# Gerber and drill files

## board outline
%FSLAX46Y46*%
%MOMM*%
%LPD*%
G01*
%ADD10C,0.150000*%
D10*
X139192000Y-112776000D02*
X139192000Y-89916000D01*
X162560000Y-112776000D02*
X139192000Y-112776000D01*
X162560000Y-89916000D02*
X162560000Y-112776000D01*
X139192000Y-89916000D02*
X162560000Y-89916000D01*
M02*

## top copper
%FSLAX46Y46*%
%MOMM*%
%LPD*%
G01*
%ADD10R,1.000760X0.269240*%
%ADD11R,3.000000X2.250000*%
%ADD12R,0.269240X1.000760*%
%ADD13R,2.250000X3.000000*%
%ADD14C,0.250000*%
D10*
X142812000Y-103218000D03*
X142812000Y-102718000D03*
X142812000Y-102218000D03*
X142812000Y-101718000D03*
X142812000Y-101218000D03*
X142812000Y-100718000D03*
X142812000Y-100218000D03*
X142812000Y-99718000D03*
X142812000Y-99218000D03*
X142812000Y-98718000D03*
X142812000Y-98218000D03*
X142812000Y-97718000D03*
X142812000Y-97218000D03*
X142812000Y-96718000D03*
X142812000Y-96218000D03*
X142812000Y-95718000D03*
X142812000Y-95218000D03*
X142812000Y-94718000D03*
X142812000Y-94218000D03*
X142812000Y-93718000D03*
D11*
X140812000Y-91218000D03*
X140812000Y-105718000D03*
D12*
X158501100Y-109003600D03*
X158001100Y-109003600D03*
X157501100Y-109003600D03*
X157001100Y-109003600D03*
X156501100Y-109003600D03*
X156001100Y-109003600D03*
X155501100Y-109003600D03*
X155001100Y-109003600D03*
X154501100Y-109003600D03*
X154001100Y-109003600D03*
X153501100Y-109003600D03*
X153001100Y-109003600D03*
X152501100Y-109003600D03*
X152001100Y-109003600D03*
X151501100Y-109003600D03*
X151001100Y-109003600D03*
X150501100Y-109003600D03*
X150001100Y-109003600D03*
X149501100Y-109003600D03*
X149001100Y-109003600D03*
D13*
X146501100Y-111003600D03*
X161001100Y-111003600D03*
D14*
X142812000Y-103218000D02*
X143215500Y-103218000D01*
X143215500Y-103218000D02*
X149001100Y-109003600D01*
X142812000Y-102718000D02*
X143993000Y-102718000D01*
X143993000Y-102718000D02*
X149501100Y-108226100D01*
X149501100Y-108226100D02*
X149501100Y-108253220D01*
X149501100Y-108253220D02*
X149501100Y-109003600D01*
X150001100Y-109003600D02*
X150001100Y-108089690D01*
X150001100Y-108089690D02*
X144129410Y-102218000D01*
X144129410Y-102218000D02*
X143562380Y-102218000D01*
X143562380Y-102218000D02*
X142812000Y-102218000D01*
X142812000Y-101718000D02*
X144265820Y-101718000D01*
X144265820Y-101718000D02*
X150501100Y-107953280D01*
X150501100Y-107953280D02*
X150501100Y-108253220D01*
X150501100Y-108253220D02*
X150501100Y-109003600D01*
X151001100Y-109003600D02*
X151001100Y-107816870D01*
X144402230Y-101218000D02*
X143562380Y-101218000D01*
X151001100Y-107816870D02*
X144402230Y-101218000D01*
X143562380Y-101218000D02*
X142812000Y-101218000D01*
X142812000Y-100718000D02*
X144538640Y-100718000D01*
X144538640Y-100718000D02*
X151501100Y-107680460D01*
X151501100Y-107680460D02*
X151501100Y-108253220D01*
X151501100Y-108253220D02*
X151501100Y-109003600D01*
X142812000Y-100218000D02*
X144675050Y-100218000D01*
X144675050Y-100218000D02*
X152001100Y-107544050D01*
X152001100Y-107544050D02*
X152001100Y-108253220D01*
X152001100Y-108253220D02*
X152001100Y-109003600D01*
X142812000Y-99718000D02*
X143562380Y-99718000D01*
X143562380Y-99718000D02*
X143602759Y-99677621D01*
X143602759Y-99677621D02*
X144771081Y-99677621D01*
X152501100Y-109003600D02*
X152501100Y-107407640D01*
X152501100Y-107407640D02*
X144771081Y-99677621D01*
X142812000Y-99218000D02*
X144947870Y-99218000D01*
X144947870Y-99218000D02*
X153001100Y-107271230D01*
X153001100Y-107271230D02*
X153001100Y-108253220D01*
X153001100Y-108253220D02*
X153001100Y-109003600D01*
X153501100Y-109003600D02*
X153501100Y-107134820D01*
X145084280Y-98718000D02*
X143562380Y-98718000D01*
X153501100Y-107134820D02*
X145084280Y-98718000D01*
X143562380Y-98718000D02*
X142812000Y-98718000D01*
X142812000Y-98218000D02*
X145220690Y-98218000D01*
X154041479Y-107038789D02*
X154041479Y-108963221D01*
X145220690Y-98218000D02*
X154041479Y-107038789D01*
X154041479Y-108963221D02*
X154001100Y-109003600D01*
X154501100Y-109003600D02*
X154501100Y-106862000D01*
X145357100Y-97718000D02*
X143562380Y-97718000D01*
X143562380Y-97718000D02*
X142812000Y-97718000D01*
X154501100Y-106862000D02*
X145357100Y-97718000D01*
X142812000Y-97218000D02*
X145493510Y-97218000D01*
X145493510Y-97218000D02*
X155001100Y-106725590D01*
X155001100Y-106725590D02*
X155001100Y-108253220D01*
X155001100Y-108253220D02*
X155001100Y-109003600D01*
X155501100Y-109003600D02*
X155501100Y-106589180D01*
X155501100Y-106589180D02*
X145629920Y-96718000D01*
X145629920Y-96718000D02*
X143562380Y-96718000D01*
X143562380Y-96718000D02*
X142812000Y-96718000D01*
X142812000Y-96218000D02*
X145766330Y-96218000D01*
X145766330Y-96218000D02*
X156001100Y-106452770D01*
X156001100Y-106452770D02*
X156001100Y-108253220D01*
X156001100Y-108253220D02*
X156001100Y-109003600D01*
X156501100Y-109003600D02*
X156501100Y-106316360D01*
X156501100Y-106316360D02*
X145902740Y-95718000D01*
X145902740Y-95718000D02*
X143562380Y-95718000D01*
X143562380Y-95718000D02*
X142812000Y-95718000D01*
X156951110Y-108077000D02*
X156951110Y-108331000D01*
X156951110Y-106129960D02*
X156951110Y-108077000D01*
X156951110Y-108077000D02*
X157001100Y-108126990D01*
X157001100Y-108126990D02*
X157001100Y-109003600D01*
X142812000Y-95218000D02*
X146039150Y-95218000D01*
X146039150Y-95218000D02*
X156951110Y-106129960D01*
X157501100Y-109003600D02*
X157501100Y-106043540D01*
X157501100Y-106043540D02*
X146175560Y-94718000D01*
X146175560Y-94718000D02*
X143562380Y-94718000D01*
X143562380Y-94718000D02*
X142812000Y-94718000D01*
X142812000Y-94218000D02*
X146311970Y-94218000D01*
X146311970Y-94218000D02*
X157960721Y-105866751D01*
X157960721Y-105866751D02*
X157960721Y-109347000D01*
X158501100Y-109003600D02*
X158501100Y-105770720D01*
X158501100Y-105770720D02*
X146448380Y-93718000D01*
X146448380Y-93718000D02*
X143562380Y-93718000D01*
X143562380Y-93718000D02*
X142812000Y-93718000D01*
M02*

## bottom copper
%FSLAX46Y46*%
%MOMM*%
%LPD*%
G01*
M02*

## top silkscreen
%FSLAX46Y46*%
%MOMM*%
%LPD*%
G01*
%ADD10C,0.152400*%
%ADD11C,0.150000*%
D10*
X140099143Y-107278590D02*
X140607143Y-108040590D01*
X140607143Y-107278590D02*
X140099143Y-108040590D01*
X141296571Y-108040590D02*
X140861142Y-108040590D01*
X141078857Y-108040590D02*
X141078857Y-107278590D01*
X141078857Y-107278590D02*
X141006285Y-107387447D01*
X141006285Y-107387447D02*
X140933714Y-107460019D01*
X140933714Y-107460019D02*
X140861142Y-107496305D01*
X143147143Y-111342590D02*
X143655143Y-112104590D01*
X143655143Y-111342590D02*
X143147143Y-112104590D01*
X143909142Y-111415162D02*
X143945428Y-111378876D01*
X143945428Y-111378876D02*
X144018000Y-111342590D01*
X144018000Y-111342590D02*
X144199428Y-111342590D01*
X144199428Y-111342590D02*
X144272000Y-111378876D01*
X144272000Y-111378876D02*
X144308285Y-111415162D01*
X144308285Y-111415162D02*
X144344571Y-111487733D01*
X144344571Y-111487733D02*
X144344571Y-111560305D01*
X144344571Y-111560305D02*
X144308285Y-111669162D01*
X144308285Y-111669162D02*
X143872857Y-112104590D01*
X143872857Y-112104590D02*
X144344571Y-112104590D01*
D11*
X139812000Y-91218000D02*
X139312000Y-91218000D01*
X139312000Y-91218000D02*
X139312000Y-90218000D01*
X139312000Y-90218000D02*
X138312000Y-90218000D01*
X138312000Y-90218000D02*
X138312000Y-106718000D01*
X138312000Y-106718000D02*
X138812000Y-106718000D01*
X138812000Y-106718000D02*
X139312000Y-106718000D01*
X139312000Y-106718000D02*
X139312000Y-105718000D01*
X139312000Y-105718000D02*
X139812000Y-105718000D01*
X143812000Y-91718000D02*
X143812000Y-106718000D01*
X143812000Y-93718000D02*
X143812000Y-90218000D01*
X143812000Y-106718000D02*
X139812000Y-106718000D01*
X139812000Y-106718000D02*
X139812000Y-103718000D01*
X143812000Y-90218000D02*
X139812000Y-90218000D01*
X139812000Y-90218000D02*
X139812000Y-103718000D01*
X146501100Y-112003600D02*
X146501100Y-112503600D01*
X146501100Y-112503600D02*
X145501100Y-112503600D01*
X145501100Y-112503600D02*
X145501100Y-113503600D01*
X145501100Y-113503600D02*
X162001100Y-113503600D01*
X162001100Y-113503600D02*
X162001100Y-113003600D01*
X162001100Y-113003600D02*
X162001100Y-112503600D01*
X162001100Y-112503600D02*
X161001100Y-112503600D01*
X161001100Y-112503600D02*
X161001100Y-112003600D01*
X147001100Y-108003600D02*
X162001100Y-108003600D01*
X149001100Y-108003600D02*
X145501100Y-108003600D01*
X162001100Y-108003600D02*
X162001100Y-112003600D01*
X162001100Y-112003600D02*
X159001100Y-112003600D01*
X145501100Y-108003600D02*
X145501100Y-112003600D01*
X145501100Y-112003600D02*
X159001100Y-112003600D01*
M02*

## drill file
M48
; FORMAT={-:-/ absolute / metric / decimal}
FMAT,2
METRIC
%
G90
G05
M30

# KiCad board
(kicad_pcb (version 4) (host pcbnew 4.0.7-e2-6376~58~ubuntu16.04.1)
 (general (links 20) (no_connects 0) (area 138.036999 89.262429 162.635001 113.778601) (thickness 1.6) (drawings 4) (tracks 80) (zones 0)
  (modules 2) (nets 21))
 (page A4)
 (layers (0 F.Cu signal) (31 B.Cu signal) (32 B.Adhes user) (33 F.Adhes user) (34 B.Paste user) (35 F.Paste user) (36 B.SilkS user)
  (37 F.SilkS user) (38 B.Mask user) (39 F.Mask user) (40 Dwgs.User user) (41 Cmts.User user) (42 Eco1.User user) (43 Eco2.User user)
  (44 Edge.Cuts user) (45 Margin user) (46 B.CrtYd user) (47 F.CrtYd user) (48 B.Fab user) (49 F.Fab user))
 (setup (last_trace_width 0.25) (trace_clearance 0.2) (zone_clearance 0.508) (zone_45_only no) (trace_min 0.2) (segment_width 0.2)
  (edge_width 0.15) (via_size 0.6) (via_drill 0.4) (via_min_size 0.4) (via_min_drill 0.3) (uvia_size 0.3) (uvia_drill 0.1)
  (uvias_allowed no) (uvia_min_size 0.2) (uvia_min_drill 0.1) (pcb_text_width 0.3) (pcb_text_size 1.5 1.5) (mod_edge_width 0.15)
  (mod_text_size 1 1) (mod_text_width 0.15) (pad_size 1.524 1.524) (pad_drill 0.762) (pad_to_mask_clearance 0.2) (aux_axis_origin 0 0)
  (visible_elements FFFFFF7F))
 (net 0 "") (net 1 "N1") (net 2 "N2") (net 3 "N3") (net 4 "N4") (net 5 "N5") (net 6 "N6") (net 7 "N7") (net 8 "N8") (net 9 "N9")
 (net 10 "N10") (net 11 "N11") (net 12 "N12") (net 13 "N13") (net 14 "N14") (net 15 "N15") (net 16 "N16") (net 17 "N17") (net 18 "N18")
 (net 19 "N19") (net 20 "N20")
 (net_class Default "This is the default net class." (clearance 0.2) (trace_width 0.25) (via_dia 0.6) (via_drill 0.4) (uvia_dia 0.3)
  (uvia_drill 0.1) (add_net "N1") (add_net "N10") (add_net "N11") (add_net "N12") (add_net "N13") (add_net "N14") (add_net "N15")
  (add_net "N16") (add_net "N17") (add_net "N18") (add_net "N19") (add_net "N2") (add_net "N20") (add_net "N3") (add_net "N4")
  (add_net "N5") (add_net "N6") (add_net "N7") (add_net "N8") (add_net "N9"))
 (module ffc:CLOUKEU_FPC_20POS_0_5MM (layer F.Cu) (at 146.812 93.218 270)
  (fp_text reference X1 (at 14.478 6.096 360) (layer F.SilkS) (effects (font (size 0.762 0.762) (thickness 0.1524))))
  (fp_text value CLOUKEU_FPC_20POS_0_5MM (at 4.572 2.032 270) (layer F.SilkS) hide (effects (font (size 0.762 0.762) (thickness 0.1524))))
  (fp_line (start -2 7) (end -2 7.5) (layer F.SilkS) (width 0.15))
  (fp_line (start -2 7.5) (end -3 7.5) (layer F.SilkS) (width 0.15))
  (fp_line (start -3 7.5) (end -3 8.5) (layer F.SilkS) (width 0.15))
  (fp_line (start -3 8.5) (end 13.5 8.5) (layer F.SilkS) (width 0.15))
  (fp_line (start 13.5 8.5) (end 13.5 8) (layer F.SilkS) (width 0.15))
  (fp_line (start 13.5 8) (end 13.5 7.5) (layer F.SilkS) (width 0.15))
  (fp_line (start 13.5 7.5) (end 12.5 7.5) (layer F.SilkS) (width 0.15))
  (fp_line (start 12.5 7.5) (end 12.5 7) (layer F.SilkS) (width 0.15))
  (fp_line (start -1.5 3) (end 13.5 3) (layer F.SilkS) (width 0.15))
  (fp_line (start 0.5 3) (end -3 3) (layer F.SilkS) (width 0.15))
  (fp_line (start 13.5 3) (end 13.5 7) (layer F.SilkS) (width 0.15))
  (fp_line (start 13.5 7) (end 10.5 7) (layer F.SilkS) (width 0.15))
  (fp_line (start -3 3) (end -3 7) (layer F.SilkS) (width 0.15))
  (fp_line (start -3 7) (end 10.5 7) (layer F.SilkS) (width 0.15))
  (pad 1 smd rect (at 10 4 90) (size 0.26924 1.00076) (layers F.Cu F.Paste F.Mask) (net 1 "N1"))
  (pad 2 smd rect (at 9.5 4 90) (size 0.26924 1.00076) (layers F.Cu F.Paste F.Mask) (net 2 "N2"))
  (pad 3 smd rect (at 9 4 90) (size 0.26924 1.00076) (layers F.Cu F.Paste F.Mask) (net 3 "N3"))
  (pad 4 smd rect (at 8.5 4 90) (size 0.26924 1.00076) (layers F.Cu F.Paste F.Mask) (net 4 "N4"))
  (pad 5 smd rect (at 8 4 90) (size 0.26924 1.00076) (layers F.Cu F.Paste F.Mask) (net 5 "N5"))
  (pad 6 smd rect (at 7.5 4 90) (size 0.26924 1.00076) (layers F.Cu F.Paste F.Mask) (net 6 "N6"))
  (pad 7 smd rect (at 7 4 90) (size 0.26924 1.00076) (layers F.Cu F.Paste F.Mask) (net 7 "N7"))
  (pad 8 smd rect (at 6.5 4 90) (size 0.26924 1.00076) (layers F.Cu F.Paste F.Mask) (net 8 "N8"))
  (pad 9 smd rect (at 6 4 90) (size 0.26924 1.00076) (layers F.Cu F.Paste F.Mask) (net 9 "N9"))
  (pad 10 smd rect (at 5.5 4 90) (size 0.26924 1.00076) (layers F.Cu F.Paste F.Mask) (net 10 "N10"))
  (pad 11 smd rect (at 5 4 90) (size 0.26924 1.00076) (layers F.Cu F.Paste F.Mask) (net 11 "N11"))
  (pad 12 smd rect (at 4.5 4 90) (size 0.26924 1.00076) (layers F.Cu F.Paste F.Mask) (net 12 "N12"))
  (pad 13 smd rect (at 4 4 90) (size 0.26924 1.00076) (layers F.Cu F.Paste F.Mask) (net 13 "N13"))
  (pad 14 smd rect (at 3.5 4 90) (size 0.26924 1.00076) (layers F.Cu F.Paste F.Mask) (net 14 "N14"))
  (pad 15 smd rect (at 3 4 90) (size 0.26924 1.00076) (layers F.Cu F.Paste F.Mask) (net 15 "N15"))
  (pad 16 smd rect (at 2.5 4 90) (size 0.26924 1.00076) (layers F.Cu F.Paste F.Mask) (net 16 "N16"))
  (pad 17 smd rect (at 2 4 90) (size 0.26924 1.00076) (layers F.Cu F.Paste F.Mask) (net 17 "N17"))
  (pad 18 smd rect (at 1.5 4 90) (size 0.26924 1.00076) (layers F.Cu F.Paste F.Mask) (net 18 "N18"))
  (pad 19 smd rect (at 1 4 90) (size 0.26924 1.00076) (layers F.Cu F.Paste F.Mask) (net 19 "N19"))
  (pad 20 smd rect (at 0.5 4 90) (size 0.26924 1.00076) (layers F.Cu F.Paste F.Mask) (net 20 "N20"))
  (pad M1 smd rect (at -2 6 270) (size 2.25 3) (layers F.Cu F.Paste F.Mask))
  (pad M2 smd rect (at 12.5 6 270) (size 2.25 3) (layers F.Cu F.Paste F.Mask)))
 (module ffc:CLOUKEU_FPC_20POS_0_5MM (layer F.Cu) (at 148.5011 105.0036)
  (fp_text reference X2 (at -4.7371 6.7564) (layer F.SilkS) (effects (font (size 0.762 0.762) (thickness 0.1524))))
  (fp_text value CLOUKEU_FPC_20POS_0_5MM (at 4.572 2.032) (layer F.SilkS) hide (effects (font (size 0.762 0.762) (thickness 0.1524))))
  (fp_line (start -2 7) (end -2 7.5) (layer F.SilkS) (width 0.15))
  (fp_line (start -2 7.5) (end -3 7.5) (layer F.SilkS) (width 0.15))
  (fp_line (start -3 7.5) (end -3 8.5) (layer F.SilkS) (width 0.15))
  (fp_line (start -3 8.5) (end 13.5 8.5) (layer F.SilkS) (width 0.15))
  (fp_line (start 13.5 8.5) (end 13.5 8) (layer F.SilkS) (width 0.15))
  (fp_line (start 13.5 8) (end 13.5 7.5) (layer F.SilkS) (width 0.15))
  (fp_line (start 13.5 7.5) (end 12.5 7.5) (layer F.SilkS) (width 0.15))
  (fp_line (start 12.5 7.5) (end 12.5 7) (layer F.SilkS) (width 0.15))
  (fp_line (start -1.5 3) (end 13.5 3) (layer F.SilkS) (width 0.15))
  (fp_line (start 0.5 3) (end -3 3) (layer F.SilkS) (width 0.15))
  (fp_line (start 13.5 3) (end 13.5 7) (layer F.SilkS) (width 0.15))
  (fp_line (start 13.5 7) (end 10.5 7) (layer F.SilkS) (width 0.15))
  (fp_line (start -3 3) (end -3 7) (layer F.SilkS) (width 0.15))
  (fp_line (start -3 7) (end 10.5 7) (layer F.SilkS) (width 0.15))
  (pad 1 smd rect (at 10 4 180) (size 0.26924 1.00076) (layers F.Cu F.Paste F.Mask) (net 20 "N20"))
  (pad 2 smd rect (at 9.5 4 180) (size 0.26924 1.00076) (layers F.Cu F.Paste F.Mask) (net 19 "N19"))
  (pad 3 smd rect (at 9 4 180) (size 0.26924 1.00076) (layers F.Cu F.Paste F.Mask) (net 18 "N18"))
  (pad 4 smd rect (at 8.5 4 180) (size 0.26924 1.00076) (layers F.Cu F.Paste F.Mask) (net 17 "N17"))
  (pad 5 smd rect (at 8 4 180) (size 0.26924 1.00076) (layers F.Cu F.Paste F.Mask) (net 16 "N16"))
  (pad 6 smd rect (at 7.5 4 180) (size 0.26924 1.00076) (layers F.Cu F.Paste F.Mask) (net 15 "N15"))
  (pad 7 smd rect (at 7 4 180) (size 0.26924 1.00076) (layers F.Cu F.Paste F.Mask) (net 14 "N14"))
  (pad 8 smd rect (at 6.5 4 180) (size 0.26924 1.00076) (layers F.Cu F.Paste F.Mask) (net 13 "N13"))
  (pad 9 smd rect (at 6 4 180) (size 0.26924 1.00076) (layers F.Cu F.Paste F.Mask) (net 12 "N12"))
  (pad 10 smd rect (at 5.5 4 180) (size 0.26924 1.00076) (layers F.Cu F.Paste F.Mask) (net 11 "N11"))
  (pad 11 smd rect (at 5 4 180) (size 0.26924 1.00076) (layers F.Cu F.Paste F.Mask) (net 10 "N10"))
  (pad 12 smd rect (at 4.5 4 180) (size 0.26924 1.00076) (layers F.Cu F.Paste F.Mask) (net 9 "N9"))
  (pad 13 smd rect (at 4 4 180) (size 0.26924 1.00076) (layers F.Cu F.Paste F.Mask) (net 8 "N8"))
  (pad 14 smd rect (at 3.5 4 180) (size 0.26924 1.00076) (layers F.Cu F.Paste F.Mask) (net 7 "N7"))
  (pad 15 smd rect (at 3 4 180) (size 0.26924 1.00076) (layers F.Cu F.Paste F.Mask) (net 6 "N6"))
  (pad 16 smd rect (at 2.5 4 180) (size 0.26924 1.00076) (layers F.Cu F.Paste F.Mask) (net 5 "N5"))
  (pad 17 smd rect (at 2 4 180) (size 0.26924 1.00076) (layers F.Cu F.Paste F.Mask) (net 4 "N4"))
  (pad 18 smd rect (at 1.5 4 180) (size 0.26924 1.00076) (layers F.Cu F.Paste F.Mask) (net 3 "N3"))
  (pad 19 smd rect (at 1 4 180) (size 0.26924 1.00076) (layers F.Cu F.Paste F.Mask) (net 2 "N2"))
  (pad 20 smd rect (at 0.5 4 180) (size 0.26924 1.00076) (layers F.Cu F.Paste F.Mask) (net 1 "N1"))
  (pad M1 smd rect (at -2 6) (size 2.25 3) (layers F.Cu F.Paste F.Mask))
  (pad M2 smd rect (at 12.5 6) (size 2.25 3) (layers F.Cu F.Paste F.Mask)))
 (gr_line (start 139.192 112.776) (end 139.192 89.916) (angle 90) (layer Edge.Cuts) (width 0.15))
 (gr_line (start 162.56 112.776) (end 139.192 112.776) (angle 90) (layer Edge.Cuts) (width 0.15))
 (gr_line (start 162.56 89.916) (end 162.56 112.776) (angle 90) (layer Edge.Cuts) (width 0.15))
 (gr_line (start 139.192 89.916) (end 162.56 89.916) (angle 90) (layer Edge.Cuts) (width 0.15))
 (segment (start 142.812 103.218) (end 143.2155 103.218) (width 0.25) (layer F.Cu) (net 1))
 (segment (start 143.2155 103.218) (end 149.0011 109.0036) (width 0.25) (layer F.Cu) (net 1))
 (segment (start 142.812 102.718) (end 143.993 102.718) (width 0.25) (layer F.Cu) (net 2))
 (segment (start 143.993 102.718) (end 149.5011 108.2261) (width 0.25) (layer F.Cu) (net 2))
 (segment (start 149.5011 108.2261) (end 149.5011 108.25322) (width 0.25) (layer F.Cu) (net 2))
 (segment (start 149.5011 108.25322) (end 149.5011 109.0036) (width 0.25) (layer F.Cu) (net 2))
 (segment (start 150.0011 109.0036) (end 150.0011 108.08969) (width 0.25) (layer F.Cu) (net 3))
 (segment (start 150.0011 108.08969) (end 144.12941 102.218) (width 0.25) (layer F.Cu) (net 3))
 (segment (start 144.12941 102.218) (end 143.56238 102.218) (width 0.25) (layer F.Cu) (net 3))
 (segment (start 143.56238 102.218) (end 142.812 102.218) (width 0.25) (layer F.Cu) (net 3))
 (segment (start 142.812 101.718) (end 144.26582 101.718) (width 0.25) (layer F.Cu) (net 4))
 (segment (start 144.26582 101.718) (end 150.5011 107.95328) (width 0.25) (layer F.Cu) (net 4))
 (segment (start 150.5011 107.95328) (end 150.5011 108.25322) (width 0.25) (layer F.Cu) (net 4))
 (segment (start 150.5011 108.25322) (end 150.5011 109.0036) (width 0.25) (layer F.Cu) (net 4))
 (segment (start 151.0011 109.0036) (end 151.0011 107.81687) (width 0.25) (layer F.Cu) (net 5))
 (segment (start 144.40223 101.218) (end 143.56238 101.218) (width 0.25) (layer F.Cu) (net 5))
 (segment (start 151.0011 107.81687) (end 144.40223 101.218) (width 0.25) (layer F.Cu) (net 5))
 (segment (start 143.56238 101.218) (end 142.812 101.218) (width 0.25) (layer F.Cu) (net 5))
 (segment (start 142.812 100.718) (end 144.53864 100.718) (width 0.25) (layer F.Cu) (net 6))
 (segment (start 144.53864 100.718) (end 151.5011 107.68046) (width 0.25) (layer F.Cu) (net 6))
 (segment (start 151.5011 107.68046) (end 151.5011 108.25322) (width 0.25) (layer F.Cu) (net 6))
 (segment (start 151.5011 108.25322) (end 151.5011 109.0036) (width 0.25) (layer F.Cu) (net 6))
 (segment (start 142.812 100.218) (end 144.67505 100.218) (width 0.25) (layer F.Cu) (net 7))
 (segment (start 144.67505 100.218) (end 152.0011 107.54405) (width 0.25) (layer F.Cu) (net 7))
 (segment (start 152.0011 107.54405) (end 152.0011 108.25322) (width 0.25) (layer F.Cu) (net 7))
 (segment (start 152.0011 108.25322) (end 152.0011 109.0036) (width 0.25) (layer F.Cu) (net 7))
 (segment (start 142.812 99.718) (end 143.56238 99.718) (width 0.25) (layer F.Cu) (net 8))
 (segment (start 143.56238 99.718) (end 143.602759 99.677621) (width 0.25) (layer F.Cu) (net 8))
 (segment (start 143.602759 99.677621) (end 144.771081 99.677621) (width 0.25) (layer F.Cu) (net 8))
 (segment (start 152.5011 109.0036) (end 152.5011 107.40764) (width 0.25) (layer F.Cu) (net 8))
 (segment (start 152.5011 107.40764) (end 144.771081 99.677621) (width 0.25) (layer F.Cu) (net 8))
 (segment (start 142.812 99.218) (end 144.94787 99.218) (width 0.25) (layer F.Cu) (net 9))
 (segment (start 144.94787 99.218) (end 153.0011 107.27123) (width 0.25) (layer F.Cu) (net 9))
 (segment (start 153.0011 107.27123) (end 153.0011 108.25322) (width 0.25) (layer F.Cu) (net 9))
 (segment (start 153.0011 108.25322) (end 153.0011 109.0036) (width 0.25) (layer F.Cu) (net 9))
 (segment (start 153.5011 109.0036) (end 153.5011 107.13482) (width 0.25) (layer F.Cu) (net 10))
 (segment (start 145.08428 98.718) (end 143.56238 98.718) (width 0.25) (layer F.Cu) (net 10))
 (segment (start 153.5011 107.13482) (end 145.08428 98.718) (width 0.25) (layer F.Cu) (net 10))
 (segment (start 143.56238 98.718) (end 142.812 98.718) (width 0.25) (layer F.Cu) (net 10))
 (segment (start 142.812 98.218) (end 145.22069 98.218) (width 0.25) (layer F.Cu) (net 11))
 (segment (start 154.041479 107.038789) (end 154.041479 108.963221) (width 0.25) (layer F.Cu) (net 11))
 (segment (start 145.22069 98.218) (end 154.041479 107.038789) (width 0.25) (layer F.Cu) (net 11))
 (segment (start 154.041479 108.963221) (end 154.0011 109.0036) (width 0.25) (layer F.Cu) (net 11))
 (segment (start 154.5011 109.0036) (end 154.5011 106.862) (width 0.25) (layer F.Cu) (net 12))
 (segment (start 145.3571 97.718) (end 143.56238 97.718) (width 0.25) (layer F.Cu) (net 12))
 (segment (start 143.56238 97.718) (end 142.812 97.718) (width 0.25) (layer F.Cu) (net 12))
 (segment (start 154.5011 106.862) (end 145.3571 97.718) (width 0.25) (layer F.Cu) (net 12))
 (segment (start 142.812 97.218) (end 145.49351 97.218) (width 0.25) (layer F.Cu) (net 13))
 (segment (start 145.49351 97.218) (end 155.0011 106.72559) (width 0.25) (layer F.Cu) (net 13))
 (segment (start 155.0011 106.72559) (end 155.0011 108.25322) (width 0.25) (layer F.Cu) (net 13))
 (segment (start 155.0011 108.25322) (end 155.0011 109.0036) (width 0.25) (layer F.Cu) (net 13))
 (segment (start 155.5011 109.0036) (end 155.5011 106.58918) (width 0.25) (layer F.Cu) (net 14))
 (segment (start 155.5011 106.58918) (end 145.62992 96.718) (width 0.25) (layer F.Cu) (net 14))
 (segment (start 145.62992 96.718) (end 143.56238 96.718) (width 0.25) (layer F.Cu) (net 14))
 (segment (start 143.56238 96.718) (end 142.812 96.718) (width 0.25) (layer F.Cu) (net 14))
 (segment (start 142.812 96.218) (end 145.76633 96.218) (width 0.25) (layer F.Cu) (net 15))
 (segment (start 145.76633 96.218) (end 156.0011 106.45277) (width 0.25) (layer F.Cu) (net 15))
 (segment (start 156.0011 106.45277) (end 156.0011 108.25322) (width 0.25) (layer F.Cu) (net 15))
 (segment (start 156.0011 108.25322) (end 156.0011 109.0036) (width 0.25) (layer F.Cu) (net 15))
 (segment (start 156.5011 109.0036) (end 156.5011 106.31636) (width 0.25) (layer F.Cu) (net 16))
 (segment (start 156.5011 106.31636) (end 145.90274 95.718) (width 0.25) (layer F.Cu) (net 16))
 (segment (start 145.90274 95.718) (end 143.56238 95.718) (width 0.25) (layer F.Cu) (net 16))
 (segment (start 143.56238 95.718) (end 142.812 95.718) (width 0.25) (layer F.Cu) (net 16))
 (segment (start 156.95111 108.077) (end 156.95111 108.331) (width 0.25) (layer F.Cu) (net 17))
 (segment (start 156.95111 106.12996) (end 156.95111 108.077) (width 0.25) (layer F.Cu) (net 17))
 (segment (start 156.95111 108.077) (end 157.0011 108.12699) (width 0.25) (layer F.Cu) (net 17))
 (segment (start 157.0011 108.12699) (end 157.0011 109.0036) (width 0.25) (layer F.Cu) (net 17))
 (segment (start 142.812 95.218) (end 146.03915 95.218) (width 0.25) (layer F.Cu) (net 17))
 (segment (start 146.03915 95.218) (end 156.95111 106.12996) (width 0.25) (layer F.Cu) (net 17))
 (segment (start 157.5011 109.0036) (end 157.5011 106.04354) (width 0.25) (layer F.Cu) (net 18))
 (segment (start 157.5011 106.04354) (end 146.17556 94.718) (width 0.25) (layer F.Cu) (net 18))
 (segment (start 146.17556 94.718) (end 143.56238 94.718) (width 0.25) (layer F.Cu) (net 18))
 (segment (start 143.56238 94.718) (end 142.812 94.718) (width 0.25) (layer F.Cu) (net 18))
 (segment (start 142.812 94.218) (end 146.31197 94.218) (width 0.25) (layer F.Cu) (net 19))
 (segment (start 146.31197 94.218) (end 157.960721 105.866751) (width 0.25) (layer F.Cu) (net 19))
 (segment (start 157.960721 105.866751) (end 157.960721 109.347) (width 0.25) (layer F.Cu) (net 19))
 (segment (start 158.5011 109.0036) (end 158.5011 105.77072) (width 0.25) (layer F.Cu) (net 20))
 (segment (start 158.5011 105.77072) (end 146.44838 93.718) (width 0.25) (layer F.Cu) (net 20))
 (segment (start 146.44838 93.718) (end 143.56238 93.718) (width 0.25) (layer F.Cu) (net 20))
 (segment (start 143.56238 93.718) (end 142.812 93.718) (width 0.25) (layer F.Cu) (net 20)))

